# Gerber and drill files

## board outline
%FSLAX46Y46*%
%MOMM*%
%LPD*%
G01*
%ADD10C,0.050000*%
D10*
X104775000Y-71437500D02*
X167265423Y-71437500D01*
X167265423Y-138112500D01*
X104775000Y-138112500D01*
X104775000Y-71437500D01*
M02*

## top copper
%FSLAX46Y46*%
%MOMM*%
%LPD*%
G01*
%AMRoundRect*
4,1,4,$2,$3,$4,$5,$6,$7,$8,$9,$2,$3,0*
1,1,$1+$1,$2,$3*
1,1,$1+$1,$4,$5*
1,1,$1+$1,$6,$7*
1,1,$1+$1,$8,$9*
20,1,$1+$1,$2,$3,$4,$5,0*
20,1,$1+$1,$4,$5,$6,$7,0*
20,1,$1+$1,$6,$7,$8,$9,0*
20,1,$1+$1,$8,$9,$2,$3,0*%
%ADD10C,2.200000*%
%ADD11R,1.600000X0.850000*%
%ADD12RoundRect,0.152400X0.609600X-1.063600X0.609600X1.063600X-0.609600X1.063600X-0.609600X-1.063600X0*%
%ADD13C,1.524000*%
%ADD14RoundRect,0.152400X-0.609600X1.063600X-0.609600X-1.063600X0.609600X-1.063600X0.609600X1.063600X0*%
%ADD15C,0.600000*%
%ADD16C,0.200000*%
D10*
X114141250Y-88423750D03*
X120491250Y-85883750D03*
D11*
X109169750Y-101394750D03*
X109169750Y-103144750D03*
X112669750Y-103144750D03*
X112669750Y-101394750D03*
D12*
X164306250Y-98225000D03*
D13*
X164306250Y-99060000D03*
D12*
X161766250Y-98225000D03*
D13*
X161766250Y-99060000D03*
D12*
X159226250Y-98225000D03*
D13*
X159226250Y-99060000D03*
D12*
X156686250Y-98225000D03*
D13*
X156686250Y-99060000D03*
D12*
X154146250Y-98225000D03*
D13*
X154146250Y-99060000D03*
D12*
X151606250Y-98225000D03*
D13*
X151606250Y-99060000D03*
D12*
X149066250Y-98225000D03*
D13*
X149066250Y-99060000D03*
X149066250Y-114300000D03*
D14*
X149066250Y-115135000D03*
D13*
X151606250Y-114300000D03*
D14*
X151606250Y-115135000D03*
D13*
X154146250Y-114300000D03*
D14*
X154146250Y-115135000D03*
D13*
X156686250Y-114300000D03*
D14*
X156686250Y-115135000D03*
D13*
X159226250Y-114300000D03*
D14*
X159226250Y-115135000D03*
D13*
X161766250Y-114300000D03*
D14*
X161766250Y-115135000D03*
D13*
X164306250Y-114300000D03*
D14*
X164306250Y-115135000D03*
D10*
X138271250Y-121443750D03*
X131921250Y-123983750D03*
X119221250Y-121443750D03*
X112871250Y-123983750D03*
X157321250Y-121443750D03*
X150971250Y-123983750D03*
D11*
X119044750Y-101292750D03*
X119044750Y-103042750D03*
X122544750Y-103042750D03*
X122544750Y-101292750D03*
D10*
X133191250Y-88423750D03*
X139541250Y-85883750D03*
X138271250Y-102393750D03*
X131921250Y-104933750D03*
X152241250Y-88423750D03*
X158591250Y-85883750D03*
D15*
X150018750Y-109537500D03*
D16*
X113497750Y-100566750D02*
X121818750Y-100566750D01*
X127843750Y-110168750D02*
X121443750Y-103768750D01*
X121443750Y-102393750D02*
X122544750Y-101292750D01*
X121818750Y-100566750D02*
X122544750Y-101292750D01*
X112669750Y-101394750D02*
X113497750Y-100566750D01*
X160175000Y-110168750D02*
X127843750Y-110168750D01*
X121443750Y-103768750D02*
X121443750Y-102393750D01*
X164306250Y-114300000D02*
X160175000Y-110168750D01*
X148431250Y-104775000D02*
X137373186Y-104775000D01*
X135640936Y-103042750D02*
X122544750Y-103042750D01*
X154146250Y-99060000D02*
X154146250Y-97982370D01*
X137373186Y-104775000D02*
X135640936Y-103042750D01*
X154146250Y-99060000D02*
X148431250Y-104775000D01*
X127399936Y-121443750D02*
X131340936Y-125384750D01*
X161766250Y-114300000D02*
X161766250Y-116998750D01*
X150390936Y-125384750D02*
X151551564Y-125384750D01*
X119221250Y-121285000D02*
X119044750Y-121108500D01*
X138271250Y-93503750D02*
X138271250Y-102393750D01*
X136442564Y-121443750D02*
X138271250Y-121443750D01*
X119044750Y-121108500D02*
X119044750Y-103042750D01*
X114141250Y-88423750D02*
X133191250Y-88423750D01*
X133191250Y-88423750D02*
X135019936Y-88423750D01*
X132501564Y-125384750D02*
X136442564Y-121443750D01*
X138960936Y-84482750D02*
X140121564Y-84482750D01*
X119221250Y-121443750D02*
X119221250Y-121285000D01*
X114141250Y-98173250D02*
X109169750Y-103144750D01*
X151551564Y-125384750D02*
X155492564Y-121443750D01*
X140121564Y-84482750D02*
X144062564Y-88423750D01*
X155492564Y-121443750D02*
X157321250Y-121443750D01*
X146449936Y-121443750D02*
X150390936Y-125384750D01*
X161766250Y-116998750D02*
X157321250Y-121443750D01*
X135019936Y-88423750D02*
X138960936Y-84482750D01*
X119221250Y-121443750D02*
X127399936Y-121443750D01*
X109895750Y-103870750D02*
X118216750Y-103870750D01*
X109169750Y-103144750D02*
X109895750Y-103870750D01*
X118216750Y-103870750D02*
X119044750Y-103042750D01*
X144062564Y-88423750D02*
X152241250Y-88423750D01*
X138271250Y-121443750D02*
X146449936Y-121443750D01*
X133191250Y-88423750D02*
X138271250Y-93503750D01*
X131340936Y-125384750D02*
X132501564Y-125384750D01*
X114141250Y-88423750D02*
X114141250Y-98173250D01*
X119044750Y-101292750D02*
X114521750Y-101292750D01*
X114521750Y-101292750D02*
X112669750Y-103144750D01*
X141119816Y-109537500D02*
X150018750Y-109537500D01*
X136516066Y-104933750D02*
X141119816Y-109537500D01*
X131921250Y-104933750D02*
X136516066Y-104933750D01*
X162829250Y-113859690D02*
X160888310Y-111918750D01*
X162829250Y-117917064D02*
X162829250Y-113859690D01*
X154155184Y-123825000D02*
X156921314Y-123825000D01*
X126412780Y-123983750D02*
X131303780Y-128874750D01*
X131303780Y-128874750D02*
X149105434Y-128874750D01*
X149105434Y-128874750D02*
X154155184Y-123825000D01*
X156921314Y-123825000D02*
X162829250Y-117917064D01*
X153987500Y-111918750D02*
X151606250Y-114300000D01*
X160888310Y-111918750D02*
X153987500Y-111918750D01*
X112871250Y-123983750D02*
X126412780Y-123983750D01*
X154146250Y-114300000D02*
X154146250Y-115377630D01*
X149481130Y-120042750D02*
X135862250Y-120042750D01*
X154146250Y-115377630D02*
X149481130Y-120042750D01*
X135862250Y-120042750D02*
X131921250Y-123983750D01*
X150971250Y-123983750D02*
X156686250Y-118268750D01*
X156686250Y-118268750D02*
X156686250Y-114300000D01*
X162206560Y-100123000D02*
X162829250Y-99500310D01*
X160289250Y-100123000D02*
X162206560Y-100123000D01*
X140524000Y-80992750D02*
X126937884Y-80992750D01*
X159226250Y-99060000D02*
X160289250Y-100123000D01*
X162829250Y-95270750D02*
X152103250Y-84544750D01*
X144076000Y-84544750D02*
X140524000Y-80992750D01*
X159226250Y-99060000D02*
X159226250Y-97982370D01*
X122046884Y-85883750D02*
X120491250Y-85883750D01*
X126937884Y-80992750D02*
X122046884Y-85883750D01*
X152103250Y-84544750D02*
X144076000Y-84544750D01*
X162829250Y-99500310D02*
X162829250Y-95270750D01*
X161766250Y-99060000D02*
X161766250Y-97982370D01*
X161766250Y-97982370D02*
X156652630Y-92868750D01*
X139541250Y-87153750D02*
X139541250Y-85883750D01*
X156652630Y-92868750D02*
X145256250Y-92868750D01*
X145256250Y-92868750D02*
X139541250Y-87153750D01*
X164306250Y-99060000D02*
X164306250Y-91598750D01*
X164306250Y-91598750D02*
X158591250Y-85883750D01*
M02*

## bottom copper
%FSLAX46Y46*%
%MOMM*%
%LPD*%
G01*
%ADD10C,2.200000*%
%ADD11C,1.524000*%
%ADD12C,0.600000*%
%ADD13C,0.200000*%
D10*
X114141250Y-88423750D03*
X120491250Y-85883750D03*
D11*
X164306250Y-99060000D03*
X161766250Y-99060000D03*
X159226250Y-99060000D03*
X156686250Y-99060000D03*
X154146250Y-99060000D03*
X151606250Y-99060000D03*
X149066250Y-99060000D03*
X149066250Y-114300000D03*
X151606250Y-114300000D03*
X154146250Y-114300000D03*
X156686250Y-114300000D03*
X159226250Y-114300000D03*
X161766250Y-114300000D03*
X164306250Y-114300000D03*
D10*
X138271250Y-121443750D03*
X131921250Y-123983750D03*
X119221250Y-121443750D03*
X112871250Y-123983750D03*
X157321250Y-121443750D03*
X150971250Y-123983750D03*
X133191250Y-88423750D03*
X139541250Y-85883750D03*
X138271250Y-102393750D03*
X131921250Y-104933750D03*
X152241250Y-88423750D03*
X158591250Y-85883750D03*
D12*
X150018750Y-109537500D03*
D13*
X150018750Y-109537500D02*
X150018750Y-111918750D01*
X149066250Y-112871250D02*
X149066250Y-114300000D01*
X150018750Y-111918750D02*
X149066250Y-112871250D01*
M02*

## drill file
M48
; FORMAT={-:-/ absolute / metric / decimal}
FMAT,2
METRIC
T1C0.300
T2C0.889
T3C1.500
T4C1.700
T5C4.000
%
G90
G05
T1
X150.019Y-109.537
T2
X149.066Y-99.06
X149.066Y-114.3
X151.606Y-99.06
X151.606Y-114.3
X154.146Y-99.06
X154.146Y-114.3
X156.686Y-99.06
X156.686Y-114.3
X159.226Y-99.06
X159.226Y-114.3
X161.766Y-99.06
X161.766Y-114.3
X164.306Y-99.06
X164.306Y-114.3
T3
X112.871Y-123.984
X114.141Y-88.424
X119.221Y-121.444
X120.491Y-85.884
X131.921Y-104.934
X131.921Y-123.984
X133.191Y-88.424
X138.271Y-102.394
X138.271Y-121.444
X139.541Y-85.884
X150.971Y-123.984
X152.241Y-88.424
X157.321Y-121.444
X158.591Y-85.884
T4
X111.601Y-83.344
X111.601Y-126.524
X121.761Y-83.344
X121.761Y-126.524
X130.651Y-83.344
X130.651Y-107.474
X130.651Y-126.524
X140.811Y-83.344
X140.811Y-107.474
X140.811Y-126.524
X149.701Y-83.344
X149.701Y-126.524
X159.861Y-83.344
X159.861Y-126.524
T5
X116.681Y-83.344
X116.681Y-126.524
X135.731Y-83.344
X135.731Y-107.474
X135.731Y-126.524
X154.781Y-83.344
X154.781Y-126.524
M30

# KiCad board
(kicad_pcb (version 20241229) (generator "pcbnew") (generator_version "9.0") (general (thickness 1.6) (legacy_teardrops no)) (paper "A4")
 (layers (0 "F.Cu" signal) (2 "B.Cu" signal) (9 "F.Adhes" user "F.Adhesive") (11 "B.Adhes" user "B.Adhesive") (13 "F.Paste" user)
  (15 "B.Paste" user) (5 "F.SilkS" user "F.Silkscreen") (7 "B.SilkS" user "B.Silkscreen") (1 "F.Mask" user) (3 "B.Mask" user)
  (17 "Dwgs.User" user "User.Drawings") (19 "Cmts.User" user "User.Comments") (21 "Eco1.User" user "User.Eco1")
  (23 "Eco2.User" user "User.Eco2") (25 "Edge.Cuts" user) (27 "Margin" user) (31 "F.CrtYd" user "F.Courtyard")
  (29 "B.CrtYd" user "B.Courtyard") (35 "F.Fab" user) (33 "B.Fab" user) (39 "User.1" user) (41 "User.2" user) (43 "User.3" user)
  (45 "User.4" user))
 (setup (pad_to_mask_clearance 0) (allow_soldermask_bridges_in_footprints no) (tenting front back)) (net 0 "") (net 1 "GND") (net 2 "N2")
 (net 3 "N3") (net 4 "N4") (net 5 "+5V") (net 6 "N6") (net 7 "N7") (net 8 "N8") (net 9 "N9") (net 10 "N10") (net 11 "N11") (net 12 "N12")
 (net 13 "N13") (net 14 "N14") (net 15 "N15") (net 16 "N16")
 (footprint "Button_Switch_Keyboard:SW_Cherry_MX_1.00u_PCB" (layer "F.Cu") (at 114.14125 88.42375 180)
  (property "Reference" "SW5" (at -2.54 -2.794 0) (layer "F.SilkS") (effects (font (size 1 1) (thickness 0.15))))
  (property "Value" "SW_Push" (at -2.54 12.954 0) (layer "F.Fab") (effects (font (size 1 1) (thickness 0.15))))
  (pad "" np_thru_hole circle (at -7.62 5.08 180) (size 1.7 1.7) (drill 1.7) (layers "*.Cu" "*.Mask"))
  (pad "" np_thru_hole circle (at -2.54 5.08 180) (size 4 4) (drill 4) (layers "*.Cu" "*.Mask"))
  (pad "" np_thru_hole circle (at 2.54 5.08 180) (size 1.7 1.7) (drill 1.7) (layers "*.Cu" "*.Mask"))
  (pad "1" thru_hole circle (at 0 0 180) (size 2.2 2.2) (drill 1.5) (layers "*.Cu" "*.Mask") (remove_unused_layers no) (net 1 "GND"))
  (pad "2" thru_hole circle (at -6.35 2.54 180) (size 2.2 2.2) (drill 1.5) (layers "*.Cu" "*.Mask") (remove_unused_layers no) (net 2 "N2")))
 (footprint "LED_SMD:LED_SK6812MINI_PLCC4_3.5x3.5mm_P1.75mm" (layer "F.Cu") (at 110.91975 102.26975)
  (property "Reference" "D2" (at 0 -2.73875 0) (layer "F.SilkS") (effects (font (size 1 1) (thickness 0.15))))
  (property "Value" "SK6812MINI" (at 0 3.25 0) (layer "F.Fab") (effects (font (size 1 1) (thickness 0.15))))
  (pad "1" smd rect (at -1.75 -0.875) (size 1.6 0.85) (layers "F.Cu" "F.Mask" "F.Paste") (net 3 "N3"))
  (pad "2" smd rect (at -1.75 0.875) (size 1.6 0.85) (layers "F.Cu" "F.Mask" "F.Paste") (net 1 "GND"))
  (pad "3" smd rect (at 1.75 0.875) (size 1.6 0.85) (layers "F.Cu" "F.Mask" "F.Paste") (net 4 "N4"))
  (pad "4" smd rect (at 1.75 -0.875) (size 1.6 0.85) (layers "F.Cu" "F.Mask" "F.Paste") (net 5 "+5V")))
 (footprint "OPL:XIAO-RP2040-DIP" (layer "F.Cu") (at 156.68625 106.68 -90)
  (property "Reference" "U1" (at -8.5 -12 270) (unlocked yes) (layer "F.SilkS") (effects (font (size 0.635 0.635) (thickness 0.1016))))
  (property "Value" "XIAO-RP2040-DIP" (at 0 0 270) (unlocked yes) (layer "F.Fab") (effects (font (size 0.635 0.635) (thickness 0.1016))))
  (pad "1" smd roundrect (at -8.455 -7.62 90) (size 2.432 1.524) (layers "F.Cu" "F.Mask") (roundrect_rratio 0.1) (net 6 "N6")
   (thermal_bridge_angle 45))
  (pad "1" thru_hole circle (at -7.62 -7.62 90) (size 1.524 1.524) (drill 0.889) (layers "*.Cu" "*.Mask") (remove_unused_layers no)
   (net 6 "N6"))
  (pad "2" smd roundrect (at -8.455 -5.08 90) (size 2.432 1.524) (layers "F.Cu" "F.Mask") (roundrect_rratio 0.1) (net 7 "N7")
   (thermal_bridge_angle 45))
  (pad "2" thru_hole circle (at -7.62 -5.08 90) (size 1.524 1.524) (drill 0.889) (layers "*.Cu" "*.Mask") (remove_unused_layers no)
   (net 7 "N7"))
  (pad "3" smd roundrect (at -8.455 -2.54 90) (size 2.432 1.524) (layers "F.Cu" "F.Mask") (roundrect_rratio 0.1) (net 2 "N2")
   (thermal_bridge_angle 45))
  (pad "3" thru_hole circle (at -7.62 -2.54 90) (size 1.524 1.524) (drill 0.889) (layers "*.Cu" "*.Mask") (remove_unused_layers no)
   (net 2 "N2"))
  (pad "4" smd roundrect (at -8.455 0 90) (size 2.432 1.524) (layers "F.Cu" "F.Mask") (roundrect_rratio 0.1) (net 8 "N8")
   (thermal_bridge_angle 45))
  (pad "4" thru_hole circle (at -7.62 0 90) (size 1.524 1.524) (drill 0.889) (layers "*.Cu" "*.Mask") (remove_unused_layers no) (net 8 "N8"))
  (pad "5" smd roundrect (at -8.455 2.54 90) (size 2.432 1.524) (layers "F.Cu" "F.Mask") (roundrect_rratio 0.1) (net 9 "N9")
   (thermal_bridge_angle 45))
  (pad "5" thru_hole circle (at -7.62 2.54 90) (size 1.524 1.524) (drill 0.889) (layers "*.Cu" "*.Mask") (remove_unused_layers no)
   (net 9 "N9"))
  (pad "6" smd roundrect (at -8.455 5.08 90) (size 2.432 1.524) (layers "F.Cu" "F.Mask") (roundrect_rratio 0.1) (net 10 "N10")
   (thermal_bridge_angle 45))
  (pad "6" thru_hole circle (at -7.62 5.08 90) (size 1.524 1.524) (drill 0.889) (layers "*.Cu" "*.Mask") (remove_unused_layers no)
   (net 10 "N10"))
  (pad "7" smd roundrect (at -8.455 7.62 90) (size 2.432 1.524) (layers "F.Cu" "F.Mask") (roundrect_rratio 0.1) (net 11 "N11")
   (thermal_bridge_angle 45))
  (pad "7" thru_hole circle (at -7.62 7.62 90) (size 1.524 1.524) (drill 0.889) (layers "*.Cu" "*.Mask") (remove_unused_layers no)
   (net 11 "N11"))
  (pad "8" thru_hole circle (at 7.62 7.62 270) (size 1.524 1.524) (drill 0.889) (layers "*.Cu" "*.Mask") (remove_unused_layers no)
   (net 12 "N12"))
  (pad "8" smd roundrect (at 8.455 7.62 270) (size 2.432 1.524) (layers "F.Cu" "F.Mask") (roundrect_rratio 0.1) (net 12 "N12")
   (thermal_bridge_angle 45))
  (pad "9" thru_hole circle (at 7.62 5.08 270) (size 1.524 1.524) (drill 0.889) (layers "*.Cu" "*.Mask") (remove_unused_layers no)
   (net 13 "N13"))
  (pad "9" smd roundrect (at 8.455 5.08 270) (size 2.432 1.524) (layers "F.Cu" "F.Mask") (roundrect_rratio 0.1) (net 13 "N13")
   (thermal_bridge_angle 45))
  (pad "10" thru_hole circle (at 7.62 2.54 270) (size 1.524 1.524) (drill 0.889) (layers "*.Cu" "*.Mask") (remove_unused_layers no)
   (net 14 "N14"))
  (pad "10" smd roundrect (at 8.455 2.54 270) (size 2.432 1.524) (layers "F.Cu" "F.Mask") (roundrect_rratio 0.1) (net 14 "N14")
   (thermal_bridge_angle 45))
  (pad "11" thru_hole circle (at 7.62 0 270) (size 1.524 1.524) (drill 0.889) (layers "*.Cu" "*.Mask") (remove_unused_layers no)
   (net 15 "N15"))
  (pad "11" smd roundrect (at 8.455 0 270) (size 2.432 1.524) (layers "F.Cu" "F.Mask") (roundrect_rratio 0.1) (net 15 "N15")
   (thermal_bridge_angle 45))
  (pad "12" thru_hole circle (at 7.62 -2.54 270) (size 1.524 1.524) (drill 0.889) (layers "*.Cu" "*.Mask") (remove_unused_layers no)
   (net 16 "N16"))
  (pad "12" smd roundrect (at 8.455 -2.54 270) (size 2.432 1.524) (layers "F.Cu" "F.Mask") (roundrect_rratio 0.1) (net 16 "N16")
   (thermal_bridge_angle 45))
  (pad "13" thru_hole circle (at 7.62 -5.08 270) (size 1.524 1.524) (drill 0.889) (layers "*.Cu" "*.Mask") (remove_unused_layers no)
   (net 1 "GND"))
  (pad "13" smd roundrect (at 8.455 -5.08 270) (size 2.432 1.524) (layers "F.Cu" "F.Mask") (roundrect_rratio 0.1) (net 1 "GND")
   (thermal_bridge_angle 45))
  (pad "14" thru_hole circle (at 7.62 -7.62 270) (size 1.524 1.524) (drill 0.889) (layers "*.Cu" "*.Mask") (remove_unused_layers no)
   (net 5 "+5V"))
  (pad "14" smd roundrect (at 8.455 -7.62 270) (size 2.432 1.524) (layers "F.Cu" "F.Mask") (roundrect_rratio 0.1) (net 5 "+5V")
   (thermal_bridge_angle 45)))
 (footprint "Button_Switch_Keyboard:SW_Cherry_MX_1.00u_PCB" (layer "F.Cu") (at 138.27125 121.44375)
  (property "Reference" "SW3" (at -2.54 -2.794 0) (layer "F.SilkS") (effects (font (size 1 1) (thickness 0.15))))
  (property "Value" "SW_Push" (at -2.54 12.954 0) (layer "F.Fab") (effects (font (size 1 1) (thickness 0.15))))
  (pad "" np_thru_hole circle (at -7.62 5.08) (size 1.7 1.7) (drill 1.7) (layers "*.Cu" "*.Mask"))
  (pad "" np_thru_hole circle (at -2.54 5.08) (size 4 4) (drill 4) (layers "*.Cu" "*.Mask"))
  (pad "" np_thru_hole circle (at 2.54 5.08) (size 1.7 1.7) (drill 1.7) (layers "*.Cu" "*.Mask"))
  (pad "1" thru_hole circle (at 0 0) (size 2.2 2.2) (drill 1.5) (layers "*.Cu" "*.Mask") (remove_unused_layers no) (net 1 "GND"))
  (pad "2" thru_hole circle (at -6.35 2.54) (size 2.2 2.2) (drill 1.5) (layers "*.Cu" "*.Mask") (remove_unused_layers no) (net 14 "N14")))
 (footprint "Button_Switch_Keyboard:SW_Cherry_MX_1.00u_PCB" (layer "F.Cu") (at 119.22125 121.44375)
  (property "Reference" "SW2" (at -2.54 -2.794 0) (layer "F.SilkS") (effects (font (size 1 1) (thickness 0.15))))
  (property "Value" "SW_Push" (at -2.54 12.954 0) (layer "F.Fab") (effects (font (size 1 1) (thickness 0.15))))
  (pad "" np_thru_hole circle (at -7.62 5.08) (size 1.7 1.7) (drill 1.7) (layers "*.Cu" "*.Mask"))
  (pad "" np_thru_hole circle (at -2.54 5.08) (size 4 4) (drill 4) (layers "*.Cu" "*.Mask"))
  (pad "" np_thru_hole circle (at 2.54 5.08) (size 1.7 1.7) (drill 1.7) (layers "*.Cu" "*.Mask"))
  (pad "1" thru_hole circle (at 0 0) (size 2.2 2.2) (drill 1.5) (layers "*.Cu" "*.Mask") (remove_unused_layers no) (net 1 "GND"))
  (pad "2" thru_hole circle (at -6.35 2.54) (size 2.2 2.2) (drill 1.5) (layers "*.Cu" "*.Mask") (remove_unused_layers no) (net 13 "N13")))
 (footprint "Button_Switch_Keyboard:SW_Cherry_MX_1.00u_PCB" (layer "F.Cu") (at 157.32125 121.44375)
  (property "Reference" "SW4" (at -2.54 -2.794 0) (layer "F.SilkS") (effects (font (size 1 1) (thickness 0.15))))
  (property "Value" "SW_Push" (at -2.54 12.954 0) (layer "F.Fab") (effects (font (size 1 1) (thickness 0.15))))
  (pad "" np_thru_hole circle (at -7.62 5.08) (size 1.7 1.7) (drill 1.7) (layers "*.Cu" "*.Mask"))
  (pad "" np_thru_hole circle (at -2.54 5.08) (size 4 4) (drill 4) (layers "*.Cu" "*.Mask"))
  (pad "" np_thru_hole circle (at 2.54 5.08) (size 1.7 1.7) (drill 1.7) (layers "*.Cu" "*.Mask"))
  (pad "1" thru_hole circle (at 0 0) (size 2.2 2.2) (drill 1.5) (layers "*.Cu" "*.Mask") (remove_unused_layers no) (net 1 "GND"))
  (pad "2" thru_hole circle (at -6.35 2.54) (size 2.2 2.2) (drill 1.5) (layers "*.Cu" "*.Mask") (remove_unused_layers no) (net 15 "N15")))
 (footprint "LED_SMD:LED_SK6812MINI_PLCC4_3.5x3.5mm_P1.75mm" (layer "F.Cu") (at 120.79475 102.16775)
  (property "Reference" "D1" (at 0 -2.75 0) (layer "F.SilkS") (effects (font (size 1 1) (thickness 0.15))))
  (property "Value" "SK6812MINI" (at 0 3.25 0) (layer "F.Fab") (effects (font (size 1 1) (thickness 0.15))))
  (pad "1" smd rect (at -1.75 -0.875) (size 1.6 0.85) (layers "F.Cu" "F.Mask" "F.Paste") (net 4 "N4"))
  (pad "2" smd rect (at -1.75 0.875) (size 1.6 0.85) (layers "F.Cu" "F.Mask" "F.Paste") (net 1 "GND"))
  (pad "3" smd rect (at 1.75 0.875) (size 1.6 0.85) (layers "F.Cu" "F.Mask" "F.Paste") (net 9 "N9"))
  (pad "4" smd rect (at 1.75 -0.875) (size 1.6 0.85) (layers "F.Cu" "F.Mask" "F.Paste") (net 5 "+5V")))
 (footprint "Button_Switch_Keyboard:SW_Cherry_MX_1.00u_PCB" (layer "F.Cu") (at 133.19125 88.42375 180)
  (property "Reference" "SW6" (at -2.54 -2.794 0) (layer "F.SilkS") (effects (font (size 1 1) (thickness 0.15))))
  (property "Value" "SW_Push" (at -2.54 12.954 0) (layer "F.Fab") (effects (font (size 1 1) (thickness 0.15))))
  (pad "" np_thru_hole circle (at -7.62 5.08 180) (size 1.7 1.7) (drill 1.7) (layers "*.Cu" "*.Mask"))
  (pad "" np_thru_hole circle (at -2.54 5.08 180) (size 4 4) (drill 4) (layers "*.Cu" "*.Mask"))
  (pad "" np_thru_hole circle (at 2.54 5.08 180) (size 1.7 1.7) (drill 1.7) (layers "*.Cu" "*.Mask"))
  (pad "1" thru_hole circle (at 0 0 180) (size 2.2 2.2) (drill 1.5) (layers "*.Cu" "*.Mask") (remove_unused_layers no) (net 1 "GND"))
  (pad "2" thru_hole circle (at -6.35 2.54 180) (size 2.2 2.2) (drill 1.5) (layers "*.Cu" "*.Mask") (remove_unused_layers no) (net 7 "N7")))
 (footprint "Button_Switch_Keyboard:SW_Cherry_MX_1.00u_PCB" (layer "F.Cu") (at 138.27125 102.39375)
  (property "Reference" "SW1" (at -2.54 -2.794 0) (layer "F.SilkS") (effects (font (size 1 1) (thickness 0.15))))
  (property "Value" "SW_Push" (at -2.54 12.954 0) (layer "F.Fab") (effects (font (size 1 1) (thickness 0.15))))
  (pad "" np_thru_hole circle (at -7.62 5.08) (size 1.7 1.7) (drill 1.7) (layers "*.Cu" "*.Mask"))
  (pad "" np_thru_hole circle (at -2.54 5.08) (size 4 4) (drill 4) (layers "*.Cu" "*.Mask"))
  (pad "" np_thru_hole circle (at 2.54 5.08) (size 1.7 1.7) (drill 1.7) (layers "*.Cu" "*.Mask"))
  (pad "1" thru_hole circle (at 0 0) (size 2.2 2.2) (drill 1.5) (layers "*.Cu" "*.Mask") (remove_unused_layers no) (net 1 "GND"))
  (pad "2" thru_hole circle (at -6.35 2.54) (size 2.2 2.2) (drill 1.5) (layers "*.Cu" "*.Mask") (remove_unused_layers no) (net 12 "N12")))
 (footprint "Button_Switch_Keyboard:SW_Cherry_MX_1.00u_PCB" (layer "F.Cu") (at 152.24125 88.42375 180)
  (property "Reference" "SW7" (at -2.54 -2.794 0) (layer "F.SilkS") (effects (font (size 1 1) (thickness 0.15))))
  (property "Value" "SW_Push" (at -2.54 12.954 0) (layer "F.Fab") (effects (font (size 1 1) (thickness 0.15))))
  (pad "" np_thru_hole circle (at -7.62 5.08 180) (size 1.7 1.7) (drill 1.7) (layers "*.Cu" "*.Mask"))
  (pad "" np_thru_hole circle (at -2.54 5.08 180) (size 4 4) (drill 4) (layers "*.Cu" "*.Mask"))
  (pad "" np_thru_hole circle (at 2.54 5.08 180) (size 1.7 1.7) (drill 1.7) (layers "*.Cu" "*.Mask"))
  (pad "1" thru_hole circle (at 0 0 180) (size 2.2 2.2) (drill 1.5) (layers "*.Cu" "*.Mask") (remove_unused_layers no) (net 1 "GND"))
  (pad "2" thru_hole circle (at -6.35 2.54 180) (size 2.2 2.2) (drill 1.5) (layers "*.Cu" "*.Mask") (remove_unused_layers no) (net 6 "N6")))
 (gr_rect (start 104.775 71.4375) (end 167.265423 138.1125) (stroke (width 0.05) (type default)) (fill no) (layer "Edge.Cuts"))
 (segment (start 113.49775 100.56675) (end 121.81875 100.56675) (width 0.2) (layer "F.Cu") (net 5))
 (segment (start 127.84375 110.16875) (end 121.44375 103.76875) (width 0.2) (layer "F.Cu") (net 5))
 (segment (start 121.44375 102.39375) (end 122.54475 101.29275) (width 0.2) (layer "F.Cu") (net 5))
 (segment (start 121.81875 100.56675) (end 122.54475 101.29275) (width 0.2) (layer "F.Cu") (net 5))
 (segment (start 112.66975 101.39475) (end 113.49775 100.56675) (width 0.2) (layer "F.Cu") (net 5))
 (segment (start 160.175 110.16875) (end 127.84375 110.16875) (width 0.2) (layer "F.Cu") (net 5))
 (segment (start 121.44375 103.76875) (end 121.44375 102.39375) (width 0.2) (layer "F.Cu") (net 5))
 (segment (start 164.30625 114.3) (end 160.175 110.16875) (width 0.2) (layer "F.Cu") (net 5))
 (segment (start 148.43125 104.775) (end 137.373186 104.775) (width 0.2) (layer "F.Cu") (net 9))
 (segment (start 135.640936 103.04275) (end 122.54475 103.04275) (width 0.2) (layer "F.Cu") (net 9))
 (segment (start 154.14625 99.06) (end 154.14625 97.98237) (width 0.2) (layer "F.Cu") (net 9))
 (segment (start 137.373186 104.775) (end 135.640936 103.04275) (width 0.2) (layer "F.Cu") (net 9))
 (segment (start 154.14625 99.06) (end 148.43125 104.775) (width 0.2) (layer "F.Cu") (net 9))
 (segment (start 127.399936 121.44375) (end 131.340936 125.38475) (width 0.2) (layer "F.Cu") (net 1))
 (segment (start 161.76625 114.3) (end 161.76625 116.99875) (width 0.2) (layer "F.Cu") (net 1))
 (segment (start 150.390936 125.38475) (end 151.551564 125.38475) (width 0.2) (layer "F.Cu") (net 1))
 (segment (start 119.22125 121.285) (end 119.04475 121.1085) (width 0.2) (layer "F.Cu") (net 1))
 (segment (start 138.27125 93.50375) (end 138.27125 102.39375) (width 0.2) (layer "F.Cu") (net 1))
 (segment (start 136.442564 121.44375) (end 138.27125 121.44375) (width 0.2) (layer "F.Cu") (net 1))
 (segment (start 119.04475 121.1085) (end 119.04475 103.04275) (width 0.2) (layer "F.Cu") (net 1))
 (segment (start 114.14125 88.42375) (end 133.19125 88.42375) (width 0.2) (layer "F.Cu") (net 1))
 (segment (start 133.19125 88.42375) (end 135.019936 88.42375) (width 0.2) (layer "F.Cu") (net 1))
 (segment (start 132.501564 125.38475) (end 136.442564 121.44375) (width 0.2) (layer "F.Cu") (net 1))
 (segment (start 138.960936 84.48275) (end 140.121564 84.48275) (width 0.2) (layer "F.Cu") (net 1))
 (segment (start 119.22125 121.44375) (end 119.22125 121.285) (width 0.2) (layer "F.Cu") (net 1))
 (segment (start 114.14125 98.17325) (end 109.16975 103.14475) (width 0.2) (layer "F.Cu") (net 1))
 (segment (start 151.551564 125.38475) (end 155.492564 121.44375) (width 0.2) (layer "F.Cu") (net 1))
 (segment (start 140.121564 84.48275) (end 144.062564 88.42375) (width 0.2) (layer "F.Cu") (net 1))
 (segment (start 155.492564 121.44375) (end 157.32125 121.44375) (width 0.2) (layer "F.Cu") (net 1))
 (segment (start 146.449936 121.44375) (end 150.390936 125.38475) (width 0.2) (layer "F.Cu") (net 1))
 (segment (start 161.76625 116.99875) (end 157.32125 121.44375) (width 0.2) (layer "F.Cu") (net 1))
 (segment (start 135.019936 88.42375) (end 138.960936 84.48275) (width 0.2) (layer "F.Cu") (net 1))
 (segment (start 119.22125 121.44375) (end 127.399936 121.44375) (width 0.2) (layer "F.Cu") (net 1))
 (segment (start 109.89575 103.87075) (end 118.21675 103.87075) (width 0.2) (layer "F.Cu") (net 1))
 (segment (start 109.16975 103.14475) (end 109.89575 103.87075) (width 0.2) (layer "F.Cu") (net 1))
 (segment (start 118.21675 103.87075) (end 119.04475 103.04275) (width 0.2) (layer "F.Cu") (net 1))
 (segment (start 144.062564 88.42375) (end 152.24125 88.42375) (width 0.2) (layer "F.Cu") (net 1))
 (segment (start 138.27125 121.44375) (end 146.449936 121.44375) (width 0.2) (layer "F.Cu") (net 1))
 (segment (start 133.19125 88.42375) (end 138.27125 93.50375) (width 0.2) (layer "F.Cu") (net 1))
 (segment (start 131.340936 125.38475) (end 132.501564 125.38475) (width 0.2) (layer "F.Cu") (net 1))
 (segment (start 114.14125 88.42375) (end 114.14125 98.17325) (width 0.2) (layer "F.Cu") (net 1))
 (segment (start 119.04475 101.29275) (end 114.52175 101.29275) (width 0.2) (layer "F.Cu") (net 4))
 (segment (start 114.52175 101.29275) (end 112.66975 103.14475) (width 0.2) (layer "F.Cu") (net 4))
 (segment (start 141.119816 109.5375) (end 150.01875 109.5375) (width 0.2) (layer "F.Cu") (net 12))
 (segment (start 136.516066 104.93375) (end 141.119816 109.5375) (width 0.2) (layer "F.Cu") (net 12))
 (segment (start 131.92125 104.93375) (end 136.516066 104.93375) (width 0.2) (layer "F.Cu") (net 12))
 (via (at 150.01875 109.5375) (size 0.6) (drill 0.3) (layers "F.Cu" "B.Cu") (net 12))
 (segment (start 150.01875 109.5375) (end 150.01875 111.91875) (width 0.2) (layer "B.Cu") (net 12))
 (segment (start 149.06625 112.87125) (end 149.06625 114.3) (width 0.2) (layer "B.Cu") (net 12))
 (segment (start 150.01875 111.91875) (end 149.06625 112.87125) (width 0.2) (layer "B.Cu") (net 12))
 (segment (start 162.82925 113.85969) (end 160.88831 111.91875) (width 0.2) (layer "F.Cu") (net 13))
 (segment (start 162.82925 117.917064) (end 162.82925 113.85969) (width 0.2) (layer "F.Cu") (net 13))
 (segment (start 154.155184 123.825) (end 156.921314 123.825) (width 0.2) (layer "F.Cu") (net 13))
 (segment (start 126.41278 123.98375) (end 131.30378 128.87475) (width 0.2) (layer "F.Cu") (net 13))
 (segment (start 131.30378 128.87475) (end 149.105434 128.87475) (width 0.2) (layer "F.Cu") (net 13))
 (segment (start 149.105434 128.87475) (end 154.155184 123.825) (width 0.2) (layer "F.Cu") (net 13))
 (segment (start 156.921314 123.825) (end 162.82925 117.917064) (width 0.2) (layer "F.Cu") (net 13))
 (segment (start 153.9875 111.91875) (end 151.60625 114.3) (width 0.2) (layer "F.Cu") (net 13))
 (segment (start 160.88831 111.91875) (end 153.9875 111.91875) (width 0.2) (layer "F.Cu") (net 13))
 (segment (start 112.87125 123.98375) (end 126.41278 123.98375) (width 0.2) (layer "F.Cu") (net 13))
 (segment (start 154.14625 114.3) (end 154.14625 115.37763) (width 0.2) (layer "F.Cu") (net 14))
 (segment (start 149.48113 120.04275) (end 135.86225 120.04275) (width 0.2) (layer "F.Cu") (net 14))
 (segment (start 154.14625 115.37763) (end 149.48113 120.04275) (width 0.2) (layer "F.Cu") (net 14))
 (segment (start 135.86225 120.04275) (end 131.92125 123.98375) (width 0.2) (layer "F.Cu") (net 14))
 (segment (start 150.97125 123.98375) (end 156.68625 118.26875) (width 0.2) (layer "F.Cu") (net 15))
 (segment (start 156.68625 118.26875) (end 156.68625 114.3) (width 0.2) (layer "F.Cu") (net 15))
 (segment (start 162.20656 100.123) (end 162.82925 99.50031) (width 0.2) (layer "F.Cu") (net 2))
 (segment (start 160.28925 100.123) (end 162.20656 100.123) (width 0.2) (layer "F.Cu") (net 2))
 (segment (start 140.524 80.99275) (end 126.937884 80.99275) (width 0.2) (layer "F.Cu") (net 2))
 (segment (start 159.22625 99.06) (end 160.28925 100.123) (width 0.2) (layer "F.Cu") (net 2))
 (segment (start 162.82925 95.27075) (end 152.10325 84.54475) (width 0.2) (layer "F.Cu") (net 2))
 (segment (start 144.076 84.54475) (end 140.524 80.99275) (width 0.2) (layer "F.Cu") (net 2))
 (segment (start 159.22625 99.06) (end 159.22625 97.98237) (width 0.2) (layer "F.Cu") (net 2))
 (segment (start 122.046884 85.88375) (end 120.49125 85.88375) (width 0.2) (layer "F.Cu") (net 2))
 (segment (start 126.937884 80.99275) (end 122.046884 85.88375) (width 0.2) (layer "F.Cu") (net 2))
 (segment (start 152.10325 84.54475) (end 144.076 84.54475) (width 0.2) (layer "F.Cu") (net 2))
 (segment (start 162.82925 99.50031) (end 162.82925 95.27075) (width 0.2) (layer "F.Cu") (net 2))
 (segment (start 161.76625 99.06) (end 161.76625 97.98237) (width 0.2) (layer "F.Cu") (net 7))
 (segment (start 161.76625 97.98237) (end 156.65263 92.86875) (width 0.2) (layer "F.Cu") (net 7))
 (segment (start 139.54125 87.15375) (end 139.54125 85.88375) (width 0.2) (layer "F.Cu") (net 7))
 (segment (start 156.65263 92.86875) (end 145.25625 92.86875) (width 0.2) (layer "F.Cu") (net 7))
 (segment (start 145.25625 92.86875) (end 139.54125 87.15375) (width 0.2) (layer "F.Cu") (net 7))
 (segment (start 164.30625 99.06) (end 164.30625 91.59875) (width 0.2) (layer "F.Cu") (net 6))
 (segment (start 164.30625 91.59875) (end 158.59125 85.88375) (width 0.2) (layer "F.Cu") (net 6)))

